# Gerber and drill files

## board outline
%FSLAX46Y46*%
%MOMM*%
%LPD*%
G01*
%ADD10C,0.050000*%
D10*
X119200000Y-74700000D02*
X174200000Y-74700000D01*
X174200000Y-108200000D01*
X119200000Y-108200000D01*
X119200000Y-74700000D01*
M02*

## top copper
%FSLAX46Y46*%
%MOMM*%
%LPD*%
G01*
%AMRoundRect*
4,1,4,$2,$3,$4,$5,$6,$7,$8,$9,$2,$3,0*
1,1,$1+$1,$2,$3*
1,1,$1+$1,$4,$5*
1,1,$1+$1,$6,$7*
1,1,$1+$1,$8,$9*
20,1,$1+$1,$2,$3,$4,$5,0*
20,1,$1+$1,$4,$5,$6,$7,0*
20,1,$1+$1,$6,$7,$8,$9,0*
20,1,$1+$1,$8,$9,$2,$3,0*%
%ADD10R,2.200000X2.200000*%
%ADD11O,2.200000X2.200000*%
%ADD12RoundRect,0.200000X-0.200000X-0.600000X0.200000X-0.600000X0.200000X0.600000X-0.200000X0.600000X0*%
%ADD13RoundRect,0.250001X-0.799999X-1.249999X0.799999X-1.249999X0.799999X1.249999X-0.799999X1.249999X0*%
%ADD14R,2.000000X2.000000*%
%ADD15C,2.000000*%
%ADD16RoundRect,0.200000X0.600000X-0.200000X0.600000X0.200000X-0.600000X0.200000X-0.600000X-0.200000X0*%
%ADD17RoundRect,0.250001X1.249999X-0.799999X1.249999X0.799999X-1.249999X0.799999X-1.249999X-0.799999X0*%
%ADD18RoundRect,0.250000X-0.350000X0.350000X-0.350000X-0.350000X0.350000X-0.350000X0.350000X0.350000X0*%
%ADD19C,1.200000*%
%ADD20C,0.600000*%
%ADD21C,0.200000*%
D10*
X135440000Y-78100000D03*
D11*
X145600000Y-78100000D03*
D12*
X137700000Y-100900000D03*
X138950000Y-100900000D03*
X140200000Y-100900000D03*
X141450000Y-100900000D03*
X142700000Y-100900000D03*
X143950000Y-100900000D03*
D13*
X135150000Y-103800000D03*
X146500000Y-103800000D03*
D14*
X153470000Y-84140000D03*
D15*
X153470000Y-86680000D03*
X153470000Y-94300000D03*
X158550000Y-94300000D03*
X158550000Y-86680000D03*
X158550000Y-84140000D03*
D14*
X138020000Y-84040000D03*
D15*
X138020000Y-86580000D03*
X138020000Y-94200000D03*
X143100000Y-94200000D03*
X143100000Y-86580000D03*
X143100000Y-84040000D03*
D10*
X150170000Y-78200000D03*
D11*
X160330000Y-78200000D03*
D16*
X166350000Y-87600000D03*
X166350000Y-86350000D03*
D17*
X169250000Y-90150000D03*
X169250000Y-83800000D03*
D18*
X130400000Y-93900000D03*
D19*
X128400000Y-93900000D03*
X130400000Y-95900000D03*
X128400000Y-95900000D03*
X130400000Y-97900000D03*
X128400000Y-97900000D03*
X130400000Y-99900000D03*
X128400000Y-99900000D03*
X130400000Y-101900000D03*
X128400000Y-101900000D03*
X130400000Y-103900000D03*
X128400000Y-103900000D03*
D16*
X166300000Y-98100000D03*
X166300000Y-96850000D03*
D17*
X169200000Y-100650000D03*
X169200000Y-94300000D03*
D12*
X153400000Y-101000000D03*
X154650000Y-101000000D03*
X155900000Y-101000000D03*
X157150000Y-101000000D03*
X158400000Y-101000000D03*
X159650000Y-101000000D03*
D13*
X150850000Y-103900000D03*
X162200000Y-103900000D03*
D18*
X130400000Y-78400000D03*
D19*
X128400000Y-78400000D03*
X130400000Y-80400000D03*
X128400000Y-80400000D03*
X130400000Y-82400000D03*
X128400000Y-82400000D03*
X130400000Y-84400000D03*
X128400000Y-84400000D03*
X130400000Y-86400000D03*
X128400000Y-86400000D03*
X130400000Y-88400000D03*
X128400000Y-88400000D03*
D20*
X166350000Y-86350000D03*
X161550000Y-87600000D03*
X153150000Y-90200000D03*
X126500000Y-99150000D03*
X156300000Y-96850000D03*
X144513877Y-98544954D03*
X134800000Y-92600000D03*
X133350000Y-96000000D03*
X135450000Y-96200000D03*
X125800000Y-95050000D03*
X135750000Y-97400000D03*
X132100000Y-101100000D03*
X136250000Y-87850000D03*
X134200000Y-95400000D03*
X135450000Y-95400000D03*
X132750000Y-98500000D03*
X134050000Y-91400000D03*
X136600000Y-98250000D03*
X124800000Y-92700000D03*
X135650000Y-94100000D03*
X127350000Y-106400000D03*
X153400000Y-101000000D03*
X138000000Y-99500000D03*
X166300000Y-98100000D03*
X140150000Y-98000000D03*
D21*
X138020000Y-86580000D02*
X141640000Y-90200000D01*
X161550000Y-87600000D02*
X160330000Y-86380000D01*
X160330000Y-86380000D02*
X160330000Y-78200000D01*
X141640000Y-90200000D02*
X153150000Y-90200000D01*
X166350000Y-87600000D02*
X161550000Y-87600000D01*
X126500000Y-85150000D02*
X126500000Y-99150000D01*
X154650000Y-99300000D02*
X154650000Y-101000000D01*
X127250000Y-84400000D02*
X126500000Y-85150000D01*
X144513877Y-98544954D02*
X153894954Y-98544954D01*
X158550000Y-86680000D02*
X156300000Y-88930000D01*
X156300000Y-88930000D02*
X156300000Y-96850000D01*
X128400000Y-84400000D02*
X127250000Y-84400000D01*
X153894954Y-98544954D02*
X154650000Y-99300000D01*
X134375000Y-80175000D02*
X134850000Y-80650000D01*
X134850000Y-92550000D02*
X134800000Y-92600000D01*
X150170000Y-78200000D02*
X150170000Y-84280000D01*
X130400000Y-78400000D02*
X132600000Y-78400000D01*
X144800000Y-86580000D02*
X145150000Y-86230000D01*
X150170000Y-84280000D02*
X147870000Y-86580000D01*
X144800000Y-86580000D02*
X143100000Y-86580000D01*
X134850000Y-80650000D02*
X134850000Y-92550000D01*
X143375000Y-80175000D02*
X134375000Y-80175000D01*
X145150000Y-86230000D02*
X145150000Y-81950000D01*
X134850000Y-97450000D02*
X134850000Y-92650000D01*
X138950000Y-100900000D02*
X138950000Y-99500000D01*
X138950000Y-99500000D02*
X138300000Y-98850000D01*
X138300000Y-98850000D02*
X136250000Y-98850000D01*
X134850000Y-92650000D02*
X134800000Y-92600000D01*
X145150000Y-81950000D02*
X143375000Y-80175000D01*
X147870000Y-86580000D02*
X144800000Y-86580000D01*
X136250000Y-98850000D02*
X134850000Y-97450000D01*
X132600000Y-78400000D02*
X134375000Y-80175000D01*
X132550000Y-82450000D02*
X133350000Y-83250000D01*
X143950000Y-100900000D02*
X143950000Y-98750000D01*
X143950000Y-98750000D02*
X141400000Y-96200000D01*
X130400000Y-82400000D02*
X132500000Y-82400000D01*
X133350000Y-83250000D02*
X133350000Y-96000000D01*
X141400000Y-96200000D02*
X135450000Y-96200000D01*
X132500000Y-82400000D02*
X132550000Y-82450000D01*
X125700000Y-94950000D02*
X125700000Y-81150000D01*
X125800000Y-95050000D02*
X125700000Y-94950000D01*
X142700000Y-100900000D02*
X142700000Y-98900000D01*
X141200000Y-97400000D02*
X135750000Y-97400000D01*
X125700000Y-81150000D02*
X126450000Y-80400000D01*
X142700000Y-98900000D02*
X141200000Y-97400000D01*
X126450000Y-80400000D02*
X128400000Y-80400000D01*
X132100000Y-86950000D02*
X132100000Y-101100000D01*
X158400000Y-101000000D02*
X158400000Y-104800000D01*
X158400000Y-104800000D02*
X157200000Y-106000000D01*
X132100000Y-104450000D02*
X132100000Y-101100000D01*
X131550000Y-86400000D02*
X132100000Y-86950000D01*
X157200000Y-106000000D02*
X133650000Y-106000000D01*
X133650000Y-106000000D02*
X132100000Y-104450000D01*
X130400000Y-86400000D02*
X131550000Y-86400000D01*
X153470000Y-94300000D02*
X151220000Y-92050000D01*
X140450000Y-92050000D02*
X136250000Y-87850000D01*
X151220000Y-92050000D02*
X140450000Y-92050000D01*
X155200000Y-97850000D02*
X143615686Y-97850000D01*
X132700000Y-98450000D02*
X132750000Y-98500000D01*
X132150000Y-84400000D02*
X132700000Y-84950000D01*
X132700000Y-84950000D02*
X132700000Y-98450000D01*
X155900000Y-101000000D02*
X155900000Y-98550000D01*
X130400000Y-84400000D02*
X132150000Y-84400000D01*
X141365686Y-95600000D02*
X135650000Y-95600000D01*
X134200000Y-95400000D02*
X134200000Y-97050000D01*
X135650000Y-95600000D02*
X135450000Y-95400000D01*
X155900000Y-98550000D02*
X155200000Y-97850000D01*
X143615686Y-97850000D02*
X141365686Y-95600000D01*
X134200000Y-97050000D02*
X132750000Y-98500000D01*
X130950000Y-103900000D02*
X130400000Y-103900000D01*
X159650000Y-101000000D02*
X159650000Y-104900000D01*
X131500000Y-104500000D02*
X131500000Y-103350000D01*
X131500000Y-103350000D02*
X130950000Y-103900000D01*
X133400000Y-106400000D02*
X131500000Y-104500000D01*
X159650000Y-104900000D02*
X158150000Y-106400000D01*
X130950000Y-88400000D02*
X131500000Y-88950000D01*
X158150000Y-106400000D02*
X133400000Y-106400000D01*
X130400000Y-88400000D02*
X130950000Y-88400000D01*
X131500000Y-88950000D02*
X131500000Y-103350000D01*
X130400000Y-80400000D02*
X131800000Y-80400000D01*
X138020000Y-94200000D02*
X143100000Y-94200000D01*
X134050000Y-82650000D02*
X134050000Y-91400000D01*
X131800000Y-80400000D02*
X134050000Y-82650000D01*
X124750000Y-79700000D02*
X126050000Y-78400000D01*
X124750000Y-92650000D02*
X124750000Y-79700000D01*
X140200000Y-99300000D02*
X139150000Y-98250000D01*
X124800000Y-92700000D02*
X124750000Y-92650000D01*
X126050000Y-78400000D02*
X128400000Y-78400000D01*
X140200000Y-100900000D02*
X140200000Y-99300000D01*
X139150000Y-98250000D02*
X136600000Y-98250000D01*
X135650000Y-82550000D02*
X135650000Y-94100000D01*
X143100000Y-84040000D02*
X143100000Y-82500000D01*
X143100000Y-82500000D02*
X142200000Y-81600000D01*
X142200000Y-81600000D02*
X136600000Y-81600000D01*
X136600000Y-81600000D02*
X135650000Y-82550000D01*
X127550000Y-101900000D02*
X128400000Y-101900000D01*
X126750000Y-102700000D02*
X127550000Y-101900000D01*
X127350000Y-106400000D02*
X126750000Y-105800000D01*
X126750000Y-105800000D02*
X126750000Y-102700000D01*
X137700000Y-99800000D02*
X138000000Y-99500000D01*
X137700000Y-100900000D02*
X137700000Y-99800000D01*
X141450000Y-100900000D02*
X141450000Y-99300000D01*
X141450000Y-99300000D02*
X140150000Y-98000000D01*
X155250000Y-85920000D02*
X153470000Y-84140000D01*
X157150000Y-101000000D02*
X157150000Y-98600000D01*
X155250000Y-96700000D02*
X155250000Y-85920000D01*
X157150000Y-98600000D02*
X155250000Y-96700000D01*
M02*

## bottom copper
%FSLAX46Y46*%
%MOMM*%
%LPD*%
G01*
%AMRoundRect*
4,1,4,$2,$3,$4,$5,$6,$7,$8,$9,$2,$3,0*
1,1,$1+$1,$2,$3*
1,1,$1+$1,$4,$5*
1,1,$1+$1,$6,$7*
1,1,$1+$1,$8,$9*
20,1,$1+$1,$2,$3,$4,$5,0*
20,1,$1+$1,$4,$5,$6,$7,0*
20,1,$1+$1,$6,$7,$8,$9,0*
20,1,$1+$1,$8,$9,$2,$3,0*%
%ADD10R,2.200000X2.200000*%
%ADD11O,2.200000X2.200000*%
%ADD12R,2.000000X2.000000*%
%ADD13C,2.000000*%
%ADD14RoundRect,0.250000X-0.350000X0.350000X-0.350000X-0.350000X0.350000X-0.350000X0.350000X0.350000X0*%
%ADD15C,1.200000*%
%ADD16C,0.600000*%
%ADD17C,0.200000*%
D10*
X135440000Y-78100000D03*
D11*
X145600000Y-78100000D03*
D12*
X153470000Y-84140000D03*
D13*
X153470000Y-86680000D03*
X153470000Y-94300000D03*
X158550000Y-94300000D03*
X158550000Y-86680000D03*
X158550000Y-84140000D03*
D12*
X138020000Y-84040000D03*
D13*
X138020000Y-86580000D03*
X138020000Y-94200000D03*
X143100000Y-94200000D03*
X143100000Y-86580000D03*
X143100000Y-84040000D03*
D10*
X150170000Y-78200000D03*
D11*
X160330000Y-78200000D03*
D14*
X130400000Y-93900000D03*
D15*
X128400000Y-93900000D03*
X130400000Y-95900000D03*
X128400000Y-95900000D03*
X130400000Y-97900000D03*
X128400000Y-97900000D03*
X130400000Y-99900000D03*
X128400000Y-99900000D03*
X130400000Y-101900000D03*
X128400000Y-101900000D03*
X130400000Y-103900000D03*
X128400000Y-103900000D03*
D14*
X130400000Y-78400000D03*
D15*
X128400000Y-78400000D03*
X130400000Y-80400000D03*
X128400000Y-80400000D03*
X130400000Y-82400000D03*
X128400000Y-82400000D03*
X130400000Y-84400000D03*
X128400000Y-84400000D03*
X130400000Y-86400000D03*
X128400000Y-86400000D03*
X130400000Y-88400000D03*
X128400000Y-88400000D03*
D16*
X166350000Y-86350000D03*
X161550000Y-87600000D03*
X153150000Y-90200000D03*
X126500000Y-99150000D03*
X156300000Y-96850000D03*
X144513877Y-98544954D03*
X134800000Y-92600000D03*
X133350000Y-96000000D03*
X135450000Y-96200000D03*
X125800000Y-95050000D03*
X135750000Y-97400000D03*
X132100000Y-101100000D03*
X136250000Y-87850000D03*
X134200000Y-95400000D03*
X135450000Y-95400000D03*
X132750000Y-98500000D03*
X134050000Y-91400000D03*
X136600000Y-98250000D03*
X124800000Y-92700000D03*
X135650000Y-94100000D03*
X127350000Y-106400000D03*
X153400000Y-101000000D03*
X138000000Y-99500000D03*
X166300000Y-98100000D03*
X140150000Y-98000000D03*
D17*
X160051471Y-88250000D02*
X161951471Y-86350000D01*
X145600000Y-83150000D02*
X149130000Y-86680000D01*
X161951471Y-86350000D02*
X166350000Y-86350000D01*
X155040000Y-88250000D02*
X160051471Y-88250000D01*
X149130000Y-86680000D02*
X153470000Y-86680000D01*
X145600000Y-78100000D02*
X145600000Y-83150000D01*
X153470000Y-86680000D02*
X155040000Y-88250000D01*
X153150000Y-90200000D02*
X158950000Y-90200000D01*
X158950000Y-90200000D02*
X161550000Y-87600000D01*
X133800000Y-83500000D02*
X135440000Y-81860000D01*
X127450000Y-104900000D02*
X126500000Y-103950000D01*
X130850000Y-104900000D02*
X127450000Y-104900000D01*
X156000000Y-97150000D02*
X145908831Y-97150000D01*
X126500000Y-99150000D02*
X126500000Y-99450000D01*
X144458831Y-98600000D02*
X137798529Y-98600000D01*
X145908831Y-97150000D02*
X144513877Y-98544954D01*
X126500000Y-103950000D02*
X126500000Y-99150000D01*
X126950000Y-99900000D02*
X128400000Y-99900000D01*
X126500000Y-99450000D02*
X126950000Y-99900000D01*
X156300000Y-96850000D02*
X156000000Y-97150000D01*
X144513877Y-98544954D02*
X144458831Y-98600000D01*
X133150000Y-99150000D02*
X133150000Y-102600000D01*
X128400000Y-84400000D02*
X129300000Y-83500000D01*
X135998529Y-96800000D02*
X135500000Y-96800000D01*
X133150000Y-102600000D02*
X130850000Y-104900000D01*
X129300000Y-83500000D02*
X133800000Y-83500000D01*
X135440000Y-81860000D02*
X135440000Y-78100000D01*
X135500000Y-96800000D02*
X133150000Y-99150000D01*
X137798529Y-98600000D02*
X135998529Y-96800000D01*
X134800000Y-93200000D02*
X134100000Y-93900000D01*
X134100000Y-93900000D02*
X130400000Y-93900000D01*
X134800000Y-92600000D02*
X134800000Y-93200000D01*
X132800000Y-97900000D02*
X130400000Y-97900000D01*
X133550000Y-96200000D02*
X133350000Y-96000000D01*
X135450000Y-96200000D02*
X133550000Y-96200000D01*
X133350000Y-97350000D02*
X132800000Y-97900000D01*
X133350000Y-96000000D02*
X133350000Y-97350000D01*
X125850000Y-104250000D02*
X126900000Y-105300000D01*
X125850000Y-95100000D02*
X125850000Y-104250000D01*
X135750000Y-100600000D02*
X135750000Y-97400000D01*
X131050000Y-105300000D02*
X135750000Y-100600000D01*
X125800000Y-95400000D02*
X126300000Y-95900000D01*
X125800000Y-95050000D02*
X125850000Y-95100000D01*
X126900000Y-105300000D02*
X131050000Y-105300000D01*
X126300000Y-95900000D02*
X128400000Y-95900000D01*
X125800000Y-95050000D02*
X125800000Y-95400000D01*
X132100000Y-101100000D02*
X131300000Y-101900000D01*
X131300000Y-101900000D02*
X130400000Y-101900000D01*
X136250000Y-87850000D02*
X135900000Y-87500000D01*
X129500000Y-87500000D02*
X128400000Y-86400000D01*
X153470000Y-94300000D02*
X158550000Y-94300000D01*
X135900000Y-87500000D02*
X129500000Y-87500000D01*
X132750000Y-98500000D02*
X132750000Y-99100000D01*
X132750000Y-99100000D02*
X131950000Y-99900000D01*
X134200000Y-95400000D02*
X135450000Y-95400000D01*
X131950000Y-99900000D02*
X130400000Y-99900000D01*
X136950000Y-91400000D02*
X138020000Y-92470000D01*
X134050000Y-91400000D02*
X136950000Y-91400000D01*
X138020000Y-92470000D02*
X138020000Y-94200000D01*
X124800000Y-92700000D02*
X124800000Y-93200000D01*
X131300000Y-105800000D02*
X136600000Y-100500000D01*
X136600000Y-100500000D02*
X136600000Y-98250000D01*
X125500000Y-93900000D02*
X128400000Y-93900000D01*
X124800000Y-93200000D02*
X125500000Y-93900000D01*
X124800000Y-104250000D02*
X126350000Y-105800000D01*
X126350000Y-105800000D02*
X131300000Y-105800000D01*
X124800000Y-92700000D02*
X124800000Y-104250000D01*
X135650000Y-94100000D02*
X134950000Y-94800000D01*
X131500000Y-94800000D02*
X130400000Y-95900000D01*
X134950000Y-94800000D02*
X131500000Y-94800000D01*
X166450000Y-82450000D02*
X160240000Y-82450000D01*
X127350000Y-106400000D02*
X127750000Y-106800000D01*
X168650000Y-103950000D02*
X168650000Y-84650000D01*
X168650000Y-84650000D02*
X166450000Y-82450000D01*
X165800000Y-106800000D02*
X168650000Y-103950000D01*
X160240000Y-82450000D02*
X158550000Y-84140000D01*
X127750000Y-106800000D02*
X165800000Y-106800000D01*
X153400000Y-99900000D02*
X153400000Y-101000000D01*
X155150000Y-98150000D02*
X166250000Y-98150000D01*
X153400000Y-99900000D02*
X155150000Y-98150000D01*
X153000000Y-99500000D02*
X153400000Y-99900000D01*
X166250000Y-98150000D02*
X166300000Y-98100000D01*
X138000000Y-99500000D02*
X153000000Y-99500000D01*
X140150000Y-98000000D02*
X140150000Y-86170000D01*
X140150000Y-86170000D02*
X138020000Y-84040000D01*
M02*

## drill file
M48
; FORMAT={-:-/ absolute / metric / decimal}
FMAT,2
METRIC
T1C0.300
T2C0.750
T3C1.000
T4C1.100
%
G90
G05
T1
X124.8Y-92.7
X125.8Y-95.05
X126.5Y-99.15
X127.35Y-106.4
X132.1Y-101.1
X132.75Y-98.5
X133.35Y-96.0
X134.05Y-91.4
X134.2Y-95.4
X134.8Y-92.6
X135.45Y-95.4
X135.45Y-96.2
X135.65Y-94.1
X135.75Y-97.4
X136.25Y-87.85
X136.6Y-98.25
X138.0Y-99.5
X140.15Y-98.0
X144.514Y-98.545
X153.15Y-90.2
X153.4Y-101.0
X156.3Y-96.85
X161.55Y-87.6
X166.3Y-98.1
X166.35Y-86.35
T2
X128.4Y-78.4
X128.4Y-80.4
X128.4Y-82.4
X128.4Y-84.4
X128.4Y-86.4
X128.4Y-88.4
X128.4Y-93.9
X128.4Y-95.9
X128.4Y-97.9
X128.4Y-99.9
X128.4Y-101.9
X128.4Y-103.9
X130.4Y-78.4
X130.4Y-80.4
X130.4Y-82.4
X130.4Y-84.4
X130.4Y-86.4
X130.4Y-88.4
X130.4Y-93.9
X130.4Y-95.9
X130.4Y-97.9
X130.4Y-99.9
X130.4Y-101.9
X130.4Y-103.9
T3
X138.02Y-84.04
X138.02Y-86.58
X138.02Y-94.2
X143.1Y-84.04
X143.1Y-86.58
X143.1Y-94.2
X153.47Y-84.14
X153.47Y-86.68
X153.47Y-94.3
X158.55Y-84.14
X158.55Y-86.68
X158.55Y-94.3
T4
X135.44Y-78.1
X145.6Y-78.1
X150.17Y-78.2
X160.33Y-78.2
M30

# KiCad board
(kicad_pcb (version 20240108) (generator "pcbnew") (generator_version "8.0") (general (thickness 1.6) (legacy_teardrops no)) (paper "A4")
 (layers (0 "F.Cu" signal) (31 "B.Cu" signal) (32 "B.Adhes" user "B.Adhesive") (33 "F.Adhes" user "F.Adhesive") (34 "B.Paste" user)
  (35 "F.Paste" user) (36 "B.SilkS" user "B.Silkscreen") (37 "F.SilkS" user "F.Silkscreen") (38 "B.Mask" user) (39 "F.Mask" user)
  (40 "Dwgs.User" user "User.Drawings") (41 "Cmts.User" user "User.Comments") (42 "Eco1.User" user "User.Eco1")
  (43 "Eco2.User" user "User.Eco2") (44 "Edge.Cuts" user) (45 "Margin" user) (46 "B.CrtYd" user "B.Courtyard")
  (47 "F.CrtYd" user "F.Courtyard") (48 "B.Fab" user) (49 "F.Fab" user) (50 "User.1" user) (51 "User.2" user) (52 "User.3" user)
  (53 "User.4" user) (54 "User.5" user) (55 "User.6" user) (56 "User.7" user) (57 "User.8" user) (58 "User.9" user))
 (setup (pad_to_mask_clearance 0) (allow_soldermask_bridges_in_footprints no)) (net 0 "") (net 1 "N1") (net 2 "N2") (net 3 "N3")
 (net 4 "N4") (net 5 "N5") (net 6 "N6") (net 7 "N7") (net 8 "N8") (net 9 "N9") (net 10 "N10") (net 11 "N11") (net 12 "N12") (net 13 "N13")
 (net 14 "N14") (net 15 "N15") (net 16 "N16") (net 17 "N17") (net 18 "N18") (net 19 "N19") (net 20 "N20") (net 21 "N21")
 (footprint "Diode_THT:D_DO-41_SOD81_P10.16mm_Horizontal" (layer "F.Cu") (at 135.44 78.1)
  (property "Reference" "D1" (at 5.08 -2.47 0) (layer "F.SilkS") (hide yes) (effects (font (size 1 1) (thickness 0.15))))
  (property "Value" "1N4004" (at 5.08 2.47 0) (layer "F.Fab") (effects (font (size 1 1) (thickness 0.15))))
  (pad "1" thru_hole rect (at 0 0) (size 2.2 2.2) (drill 1.1) (layers "*.Cu" "*.Mask") (remove_unused_layers no) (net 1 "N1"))
  (pad "2" thru_hole oval (at 10.16 0) (size 2.2 2.2) (drill 1.1) (layers "*.Cu" "*.Mask") (remove_unused_layers no) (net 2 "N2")))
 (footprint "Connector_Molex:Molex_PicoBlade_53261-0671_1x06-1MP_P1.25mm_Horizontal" (layer "F.Cu") (at 140.825 103.3)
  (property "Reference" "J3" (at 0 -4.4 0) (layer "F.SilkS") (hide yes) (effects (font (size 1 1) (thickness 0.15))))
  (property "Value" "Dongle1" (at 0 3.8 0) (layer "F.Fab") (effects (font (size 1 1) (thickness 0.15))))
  (pad "1" smd roundrect (at -3.125 -2.4) (size 0.8 1.6) (layers "F.Cu" "F.Paste" "F.Mask") (roundrect_rratio 0.25) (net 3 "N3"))
  (pad "2" smd roundrect (at -1.875 -2.4) (size 0.8 1.6) (layers "F.Cu" "F.Paste" "F.Mask") (roundrect_rratio 0.25) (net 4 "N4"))
  (pad "3" smd roundrect (at -0.625 -2.4) (size 0.8 1.6) (layers "F.Cu" "F.Paste" "F.Mask") (roundrect_rratio 0.25) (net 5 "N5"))
  (pad "4" smd roundrect (at 0.625 -2.4) (size 0.8 1.6) (layers "F.Cu" "F.Paste" "F.Mask") (roundrect_rratio 0.25) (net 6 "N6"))
  (pad "5" smd roundrect (at 1.875 -2.4) (size 0.8 1.6) (layers "F.Cu" "F.Paste" "F.Mask") (roundrect_rratio 0.25) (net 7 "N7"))
  (pad "6" smd roundrect (at 3.125 -2.4) (size 0.8 1.6) (layers "F.Cu" "F.Paste" "F.Mask") (roundrect_rratio 0.25) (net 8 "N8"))
  (pad "MP" smd roundrect (at -5.675 0.5) (size 2.1 3) (layers "F.Cu" "F.Paste" "F.Mask") (roundrect_rratio 0.119048))
  (pad "MP" smd roundrect (at 5.675 0.5) (size 2.1 3) (layers "F.Cu" "F.Paste" "F.Mask") (roundrect_rratio 0.119048)))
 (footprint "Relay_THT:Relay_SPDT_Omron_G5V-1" (layer "F.Cu") (at 153.47 84.14)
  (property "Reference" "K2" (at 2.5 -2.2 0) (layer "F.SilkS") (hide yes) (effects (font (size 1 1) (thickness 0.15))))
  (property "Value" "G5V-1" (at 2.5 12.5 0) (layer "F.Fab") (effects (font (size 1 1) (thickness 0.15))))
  (pad "1" thru_hole rect (at 0 0) (size 2 2) (drill 1) (layers "*.Cu" "*.Mask") (remove_unused_layers no) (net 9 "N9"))
  (pad "2" thru_hole circle (at 0 2.54) (size 2 2) (drill 1) (layers "*.Cu" "*.Mask") (remove_unused_layers no) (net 2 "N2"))
  (pad "5" thru_hole circle (at 0 10.16) (size 2 2) (drill 1) (layers "*.Cu" "*.Mask") (remove_unused_layers no) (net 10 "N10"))
  (pad "6" thru_hole circle (at 5.08 10.16) (size 2 2) (drill 1) (layers "*.Cu" "*.Mask") (remove_unused_layers no) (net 10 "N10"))
  (pad "9" thru_hole circle (at 5.08 2.54) (size 2 2) (drill 1) (layers "*.Cu" "*.Mask") (remove_unused_layers no) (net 1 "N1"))
  (pad "10" thru_hole circle (at 5.08 0) (size 2 2) (drill 1) (layers "*.Cu" "*.Mask") (remove_unused_layers no) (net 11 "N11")))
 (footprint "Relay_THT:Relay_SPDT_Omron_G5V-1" (layer "F.Cu") (at 138.02 84.04)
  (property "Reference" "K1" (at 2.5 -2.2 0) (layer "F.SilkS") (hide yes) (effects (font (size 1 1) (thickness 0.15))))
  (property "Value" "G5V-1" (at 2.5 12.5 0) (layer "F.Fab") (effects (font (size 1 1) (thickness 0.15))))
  (pad "1" thru_hole rect (at 0 0) (size 2 2) (drill 1) (layers "*.Cu" "*.Mask") (remove_unused_layers no) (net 6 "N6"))
  (pad "2" thru_hole circle (at 0 2.54) (size 2 2) (drill 1) (layers "*.Cu" "*.Mask") (remove_unused_layers no) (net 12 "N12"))
  (pad "5" thru_hole circle (at 0 10.16) (size 2 2) (drill 1) (layers "*.Cu" "*.Mask") (remove_unused_layers no) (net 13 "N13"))
  (pad "6" thru_hole circle (at 5.08 10.16) (size 2 2) (drill 1) (layers "*.Cu" "*.Mask") (remove_unused_layers no) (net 13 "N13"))
  (pad "9" thru_hole circle (at 5.08 2.54) (size 2 2) (drill 1) (layers "*.Cu" "*.Mask") (remove_unused_layers no) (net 4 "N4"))
  (pad "10" thru_hole circle (at 5.08 0) (size 2 2) (drill 1) (layers "*.Cu" "*.Mask") (remove_unused_layers no) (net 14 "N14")))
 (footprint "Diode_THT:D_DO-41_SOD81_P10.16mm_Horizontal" (layer "F.Cu") (at 150.17 78.2)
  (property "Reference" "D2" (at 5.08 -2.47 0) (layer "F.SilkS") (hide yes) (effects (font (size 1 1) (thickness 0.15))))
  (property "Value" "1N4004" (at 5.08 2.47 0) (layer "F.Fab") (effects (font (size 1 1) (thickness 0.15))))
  (pad "1" thru_hole rect (at 0 0) (size 2.2 2.2) (drill 1.1) (layers "*.Cu" "*.Mask") (remove_unused_layers no) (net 4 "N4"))
  (pad "2" thru_hole oval (at 10.16 0) (size 2.2 2.2) (drill 1.1) (layers "*.Cu" "*.Mask") (remove_unused_layers no) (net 12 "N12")))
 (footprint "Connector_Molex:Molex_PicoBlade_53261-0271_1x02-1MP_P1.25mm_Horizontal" (layer "F.Cu") (at 168.75 86.975 90)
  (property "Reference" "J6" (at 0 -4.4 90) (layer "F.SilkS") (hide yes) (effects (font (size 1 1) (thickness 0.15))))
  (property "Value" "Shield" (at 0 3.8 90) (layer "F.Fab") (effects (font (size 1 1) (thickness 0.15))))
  (pad "1" smd roundrect (at -0.625 -2.4 90) (size 0.8 1.6) (layers "F.Cu" "F.Paste" "F.Mask") (roundrect_rratio 0.25) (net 12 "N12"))
  (pad "2" smd roundrect (at 0.625 -2.4 90) (size 0.8 1.6) (layers "F.Cu" "F.Paste" "F.Mask") (roundrect_rratio 0.25) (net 2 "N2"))
  (pad "MP" smd roundrect (at -3.175 0.5 90) (size 2.1 3) (layers "F.Cu" "F.Paste" "F.Mask") (roundrect_rratio 0.119048))
  (pad "MP" smd roundrect (at 3.175 0.5 90) (size 2.1 3) (layers "F.Cu" "F.Paste" "F.Mask") (roundrect_rratio 0.119048)))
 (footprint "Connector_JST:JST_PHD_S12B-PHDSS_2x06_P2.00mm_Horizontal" (layer "F.Cu") (at 130.4 93.9 -90)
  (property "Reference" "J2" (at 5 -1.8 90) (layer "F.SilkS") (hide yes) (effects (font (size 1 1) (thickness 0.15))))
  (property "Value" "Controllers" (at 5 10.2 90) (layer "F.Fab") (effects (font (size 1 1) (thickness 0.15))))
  (pad "1" thru_hole roundrect (at 0 0 270) (size 1.2 1.2) (drill 0.75) (layers "*.Cu" "*.Mask") (remove_unused_layers no)
   (roundrect_rratio 0.208333) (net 4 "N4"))
  (pad "2" thru_hole circle (at 0 2 270) (size 1.2 1.2) (drill 0.75) (layers "*.Cu" "*.Mask") (remove_unused_layers no) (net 5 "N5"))
  (pad "3" thru_hole circle (at 2 0 270) (size 1.2 1.2) (drill 0.75) (layers "*.Cu" "*.Mask") (remove_unused_layers no) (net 14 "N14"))
  (pad "4" thru_hole circle (at 2 2 270) (size 1.2 1.2) (drill 0.75) (layers "*.Cu" "*.Mask") (remove_unused_layers no) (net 7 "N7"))
  (pad "5" thru_hole circle (at 4 0 270) (size 1.2 1.2) (drill 0.75) (layers "*.Cu" "*.Mask") (remove_unused_layers no) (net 8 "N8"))
  (pad "6" thru_hole circle (at 4 2 270) (size 1.2 1.2) (drill 0.75) (layers "*.Cu" "*.Mask") (remove_unused_layers no) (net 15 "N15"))
  (pad "7" thru_hole circle (at 6 0 270) (size 1.2 1.2) (drill 0.75) (layers "*.Cu" "*.Mask") (remove_unused_layers no) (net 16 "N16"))
  (pad "8" thru_hole circle (at 6 2 270) (size 1.2 1.2) (drill 0.75) (layers "*.Cu" "*.Mask") (remove_unused_layers no) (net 1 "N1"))
  (pad "9" thru_hole circle (at 8 0 270) (size 1.2 1.2) (drill 0.75) (layers "*.Cu" "*.Mask") (remove_unused_layers no) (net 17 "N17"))
  (pad "10" thru_hole circle (at 8 2 270) (size 1.2 1.2) (drill 0.75) (layers "*.Cu" "*.Mask") (remove_unused_layers no) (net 11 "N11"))
  (pad "11" thru_hole circle (at 10 0 270) (size 1.2 1.2) (drill 0.75) (layers "*.Cu" "*.Mask") (remove_unused_layers no) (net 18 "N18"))
  (pad "12" thru_hole circle (at 10 2 270) (size 1.2 1.2) (drill 0.75) (layers "*.Cu" "*.Mask") (remove_unused_layers no) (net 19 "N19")))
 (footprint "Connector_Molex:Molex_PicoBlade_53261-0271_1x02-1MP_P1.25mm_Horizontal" (layer "F.Cu") (at 168.7 97.475 90)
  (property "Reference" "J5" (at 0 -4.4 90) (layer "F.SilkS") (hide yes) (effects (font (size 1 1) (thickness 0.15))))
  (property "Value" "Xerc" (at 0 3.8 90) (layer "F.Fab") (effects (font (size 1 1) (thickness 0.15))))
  (pad "1" smd roundrect (at -0.625 -2.4 90) (size 0.8 1.6) (layers "F.Cu" "F.Paste" "F.Mask") (roundrect_rratio 0.25) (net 3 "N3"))
  (pad "2" smd roundrect (at 0.625 -2.4 90) (size 0.8 1.6) (layers "F.Cu" "F.Paste" "F.Mask") (roundrect_rratio 0.25))
  (pad "MP" smd roundrect (at -3.175 0.5 90) (size 2.1 3) (layers "F.Cu" "F.Paste" "F.Mask") (roundrect_rratio 0.119048))
  (pad "MP" smd roundrect (at 3.175 0.5 90) (size 2.1 3) (layers "F.Cu" "F.Paste" "F.Mask") (roundrect_rratio 0.119048)))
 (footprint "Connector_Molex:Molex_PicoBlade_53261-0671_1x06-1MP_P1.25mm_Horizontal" (layer "F.Cu") (at 156.525 103.4)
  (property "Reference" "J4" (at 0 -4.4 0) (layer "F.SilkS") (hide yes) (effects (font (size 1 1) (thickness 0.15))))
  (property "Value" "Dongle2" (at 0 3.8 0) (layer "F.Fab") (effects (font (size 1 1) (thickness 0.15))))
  (pad "1" smd roundrect (at -3.125 -2.4) (size 0.8 1.6) (layers "F.Cu" "F.Paste" "F.Mask") (roundrect_rratio 0.25) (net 3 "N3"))
  (pad "2" smd roundrect (at -1.875 -2.4) (size 0.8 1.6) (layers "F.Cu" "F.Paste" "F.Mask") (roundrect_rratio 0.25) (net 1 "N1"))
  (pad "3" smd roundrect (at -0.625 -2.4) (size 0.8 1.6) (layers "F.Cu" "F.Paste" "F.Mask") (roundrect_rratio 0.25) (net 16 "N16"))
  (pad "4" smd roundrect (at 0.625 -2.4) (size 0.8 1.6) (layers "F.Cu" "F.Paste" "F.Mask") (roundrect_rratio 0.25) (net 9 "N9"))
  (pad "5" smd roundrect (at 1.875 -2.4) (size 0.8 1.6) (layers "F.Cu" "F.Paste" "F.Mask") (roundrect_rratio 0.25) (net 17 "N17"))
  (pad "6" smd roundrect (at 3.125 -2.4) (size 0.8 1.6) (layers "F.Cu" "F.Paste" "F.Mask") (roundrect_rratio 0.25) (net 18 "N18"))
  (pad "MP" smd roundrect (at -5.675 0.5) (size 2.1 3) (layers "F.Cu" "F.Paste" "F.Mask") (roundrect_rratio 0.119048))
  (pad "MP" smd roundrect (at 5.675 0.5) (size 2.1 3) (layers "F.Cu" "F.Paste" "F.Mask") (roundrect_rratio 0.119048)))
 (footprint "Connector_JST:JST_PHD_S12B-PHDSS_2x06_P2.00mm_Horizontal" (layer "F.Cu") (at 130.4 78.4 -90)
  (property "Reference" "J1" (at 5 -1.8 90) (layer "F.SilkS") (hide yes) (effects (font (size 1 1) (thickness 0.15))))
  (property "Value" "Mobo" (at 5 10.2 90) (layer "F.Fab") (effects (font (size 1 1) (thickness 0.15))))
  (pad "1" thru_hole roundrect (at 0 0 270) (size 1.2 1.2) (drill 0.75) (layers "*.Cu" "*.Mask") (remove_unused_layers no)
   (roundrect_rratio 0.208333) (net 4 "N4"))
  (pad "2" thru_hole circle (at 0 2 270) (size 1.2 1.2) (drill 0.75) (layers "*.Cu" "*.Mask") (remove_unused_layers no) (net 5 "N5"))
  (pad "3" thru_hole circle (at 2 0 270) (size 1.2 1.2) (drill 0.75) (layers "*.Cu" "*.Mask") (remove_unused_layers no) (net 13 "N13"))
  (pad "4" thru_hole circle (at 2 2 270) (size 1.2 1.2) (drill 0.75) (layers "*.Cu" "*.Mask") (remove_unused_layers no) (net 7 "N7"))
  (pad "5" thru_hole circle (at 4 0 270) (size 1.2 1.2) (drill 0.75) (layers "*.Cu" "*.Mask") (remove_unused_layers no) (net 8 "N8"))
  (pad "6" thru_hole circle (at 4 2 270) (size 1.2 1.2) (drill 0.75) (layers "*.Cu" "*.Mask") (remove_unused_layers no) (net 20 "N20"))
  (pad "7" thru_hole circle (at 6 0 270) (size 1.2 1.2) (drill 0.75) (layers "*.Cu" "*.Mask") (remove_unused_layers no) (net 16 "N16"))
  (pad "8" thru_hole circle (at 6 2 270) (size 1.2 1.2) (drill 0.75) (layers "*.Cu" "*.Mask") (remove_unused_layers no) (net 1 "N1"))
  (pad "9" thru_hole circle (at 8 0 270) (size 1.2 1.2) (drill 0.75) (layers "*.Cu" "*.Mask") (remove_unused_layers no) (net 17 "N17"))
  (pad "10" thru_hole circle (at 8 2 270) (size 1.2 1.2) (drill 0.75) (layers "*.Cu" "*.Mask") (remove_unused_layers no) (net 10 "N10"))
  (pad "11" thru_hole circle (at 10 0 270) (size 1.2 1.2) (drill 0.75) (layers "*.Cu" "*.Mask") (remove_unused_layers no) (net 18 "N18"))
  (pad "12" thru_hole circle (at 10 2 270) (size 1.2 1.2) (drill 0.75) (layers "*.Cu" "*.Mask") (remove_unused_layers no) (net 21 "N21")))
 (gr_rect (start 119.2 74.7) (end 174.2 108.2) (stroke (width 0.05) (type default)) (fill none) (layer "Edge.Cuts"))
 (via (at 166.35 86.35) (size 0.6) (drill 0.3) (layers "F.Cu" "B.Cu") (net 2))
 (segment (start 160.051471 88.25) (end 161.951471 86.35) (width 0.2) (layer "B.Cu") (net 2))
 (segment (start 145.6 83.15) (end 149.13 86.68) (width 0.2) (layer "B.Cu") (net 2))
 (segment (start 161.951471 86.35) (end 166.35 86.35) (width 0.2) (layer "B.Cu") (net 2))
 (segment (start 155.04 88.25) (end 160.051471 88.25) (width 0.2) (layer "B.Cu") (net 2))
 (segment (start 149.13 86.68) (end 153.47 86.68) (width 0.2) (layer "B.Cu") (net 2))
 (segment (start 145.6 78.1) (end 145.6 83.15) (width 0.2) (layer "B.Cu") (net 2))
 (segment (start 153.47 86.68) (end 155.04 88.25) (width 0.2) (layer "B.Cu") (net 2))
 (segment (start 138.02 86.58) (end 141.64 90.2) (width 0.2) (layer "F.Cu") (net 12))
 (segment (start 161.55 87.6) (end 160.33 86.38) (width 0.2) (layer "F.Cu") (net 12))
 (segment (start 160.33 86.38) (end 160.33 78.2) (width 0.2) (layer "F.Cu") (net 12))
 (segment (start 141.64 90.2) (end 153.15 90.2) (width 0.2) (layer "F.Cu") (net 12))
 (segment (start 166.35 87.6) (end 161.55 87.6) (width 0.2) (layer "F.Cu") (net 12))
 (via (at 161.55 87.6) (size 0.6) (drill 0.3) (layers "F.Cu" "B.Cu") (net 12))
 (via (at 153.15 90.2) (size 0.6) (drill 0.3) (layers "F.Cu" "B.Cu") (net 12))
 (segment (start 153.15 90.2) (end 158.95 90.2) (width 0.2) (layer "B.Cu") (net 12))
 (segment (start 158.95 90.2) (end 161.55 87.6) (width 0.2) (layer "B.Cu") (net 12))
 (segment (start 126.5 85.15) (end 126.5 99.15) (width 0.2) (layer "F.Cu") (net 1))
 (segment (start 154.65 99.3) (end 154.65 101) (width 0.2) (layer "F.Cu") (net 1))
 (segment (start 127.25 84.4) (end 126.5 85.15) (width 0.2) (layer "F.Cu") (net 1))
 (segment (start 144.513877 98.544954) (end 153.894954 98.544954) (width 0.2) (layer "F.Cu") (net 1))
 (segment (start 158.55 86.68) (end 156.3 88.93) (width 0.2) (layer "F.Cu") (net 1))
 (segment (start 156.3 88.93) (end 156.3 96.85) (width 0.2) (layer "F.Cu") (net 1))
 (segment (start 128.4 84.4) (end 127.25 84.4) (width 0.2) (layer "F.Cu") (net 1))
 (segment (start 153.894954 98.544954) (end 154.65 99.3) (width 0.2) (layer "F.Cu") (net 1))
 (via (at 126.5 99.15) (size 0.6) (drill 0.3) (layers "F.Cu" "B.Cu") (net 1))
 (via (at 156.3 96.85) (size 0.6) (drill 0.3) (layers "F.Cu" "B.Cu") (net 1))
 (via (at 144.513877 98.544954) (size 0.6) (drill 0.3) (layers "F.Cu" "B.Cu") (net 1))
 (segment (start 133.8 83.5) (end 135.44 81.86) (width 0.2) (layer "B.Cu") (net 1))
 (segment (start 127.45 104.9) (end 126.5 103.95) (width 0.2) (layer "B.Cu") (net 1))
 (segment (start 130.85 104.9) (end 127.45 104.9) (width 0.2) (layer "B.Cu") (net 1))
 (segment (start 156 97.15) (end 145.908831 97.15) (width 0.2) (layer "B.Cu") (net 1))
 (segment (start 126.5 99.15) (end 126.5 99.45) (width 0.2) (layer "B.Cu") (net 1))
 (segment (start 144.458831 98.6) (end 137.798529 98.6) (width 0.2) (layer "B.Cu") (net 1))
 (segment (start 145.908831 97.15) (end 144.513877 98.544954) (width 0.2) (layer "B.Cu") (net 1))
 (segment (start 126.5 103.95) (end 126.5 99.15) (width 0.2) (layer "B.Cu") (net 1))
 (segment (start 126.95 99.9) (end 128.4 99.9) (width 0.2) (layer "B.Cu") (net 1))
 (segment (start 126.5 99.45) (end 126.95 99.9) (width 0.2) (layer "B.Cu") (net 1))
 (segment (start 156.3 96.85) (end 156 97.15) (width 0.2) (layer "B.Cu") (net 1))
 (segment (start 144.513877 98.544954) (end 144.458831 98.6) (width 0.2) (layer "B.Cu") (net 1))
 (segment (start 133.15 99.15) (end 133.15 102.6) (width 0.2) (layer "B.Cu") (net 1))
 (segment (start 128.4 84.4) (end 129.3 83.5) (width 0.2) (layer "B.Cu") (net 1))
 (segment (start 135.998529 96.8) (end 135.5 96.8) (width 0.2) (layer "B.Cu") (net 1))
 (segment (start 133.15 102.6) (end 130.85 104.9) (width 0.2) (layer "B.Cu") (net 1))
 (segment (start 129.3 83.5) (end 133.8 83.5) (width 0.2) (layer "B.Cu") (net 1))
 (segment (start 135.44 81.86) (end 135.44 78.1) (width 0.2) (layer "B.Cu") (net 1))
 (segment (start 135.5 96.8) (end 133.15 99.15) (width 0.2) (layer "B.Cu") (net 1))
 (segment (start 137.798529 98.6) (end 135.998529 96.8) (width 0.2) (layer "B.Cu") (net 1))
 (segment (start 134.375 80.175) (end 134.85 80.65) (width 0.2) (layer "F.Cu") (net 4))
 (segment (start 134.85 92.55) (end 134.8 92.6) (width 0.2) (layer "F.Cu") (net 4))
 (segment (start 150.17 78.2) (end 150.17 84.28) (width 0.2) (layer "F.Cu") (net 4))
 (segment (start 130.4 78.4) (end 132.6 78.4) (width 0.2) (layer "F.Cu") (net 4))
 (segment (start 144.8 86.58) (end 145.15 86.23) (width 0.2) (layer "F.Cu") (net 4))
 (segment (start 150.17 84.28) (end 147.87 86.58) (width 0.2) (layer "F.Cu") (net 4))
 (segment (start 144.8 86.58) (end 143.1 86.58) (width 0.2) (layer "F.Cu") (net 4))
 (segment (start 134.85 80.65) (end 134.85 92.55) (width 0.2) (layer "F.Cu") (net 4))
 (segment (start 143.375 80.175) (end 134.375 80.175) (width 0.2) (layer "F.Cu") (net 4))
 (segment (start 145.15 86.23) (end 145.15 81.95) (width 0.2) (layer "F.Cu") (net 4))
 (segment (start 134.85 97.45) (end 134.85 92.65) (width 0.2) (layer "F.Cu") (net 4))
 (segment (start 138.95 100.9) (end 138.95 99.5) (width 0.2) (layer "F.Cu") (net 4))
 (segment (start 138.95 99.5) (end 138.3 98.85) (width 0.2) (layer "F.Cu") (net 4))
 (segment (start 138.3 98.85) (end 136.25 98.85) (width 0.2) (layer "F.Cu") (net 4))
 (segment (start 134.85 92.65) (end 134.8 92.6) (width 0.2) (layer "F.Cu") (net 4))
 (segment (start 145.15 81.95) (end 143.375 80.175) (width 0.2) (layer "F.Cu") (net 4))
 (segment (start 147.87 86.58) (end 144.8 86.58) (width 0.2) (layer "F.Cu") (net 4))
 (segment (start 136.25 98.85) (end 134.85 97.45) (width 0.2) (layer "F.Cu") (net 4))
 (segment (start 132.6 78.4) (end 134.375 80.175) (width 0.2) (layer "F.Cu") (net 4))
 (via (at 134.8 92.6) (size 0.6) (drill 0.3) (layers "F.Cu" "B.Cu") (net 4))
 (segment (start 134.8 93.2) (end 134.1 93.9) (width 0.2) (layer "B.Cu") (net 4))
 (segment (start 134.1 93.9) (end 130.4 93.9) (width 0.2) (layer "B.Cu") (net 4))
 (segment (start 134.8 92.6) (end 134.8 93.2) (width 0.2) (layer "B.Cu") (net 4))
 (segment (start 132.55 82.45) (end 133.35 83.25) (width 0.2) (layer "F.Cu") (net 8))
 (segment (start 143.95 100.9) (end 143.95 98.75) (width 0.2) (layer "F.Cu") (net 8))
 (segment (start 143.95 98.75) (end 141.4 96.2) (width 0.2) (layer "F.Cu") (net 8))
 (segment (start 130.4 82.4) (end 132.5 82.4) (width 0.2) (layer "F.Cu") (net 8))
 (segment (start 133.35 83.25) (end 133.35 96) (width 0.2) (layer "F.Cu") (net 8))
 (segment (start 141.4 96.2) (end 135.45 96.2) (width 0.2) (layer "F.Cu") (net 8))
 (segment (start 132.5 82.4) (end 132.55 82.45) (width 0.2) (layer "F.Cu") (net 8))
 (via (at 133.35 96) (size 0.6) (drill 0.3) (layers "F.Cu" "B.Cu") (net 8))
 (via (at 135.45 96.2) (size 0.6) (drill 0.3) (layers "F.Cu" "B.Cu") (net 8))
 (segment (start 132.8 97.9) (end 130.4 97.9) (width 0.2) (layer "B.Cu") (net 8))
 (segment (start 133.55 96.2) (end 133.35 96) (width 0.2) (layer "B.Cu") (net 8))
 (segment (start 135.45 96.2) (end 133.55 96.2) (width 0.2) (layer "B.Cu") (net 8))
 (segment (start 133.35 97.35) (end 132.8 97.9) (width 0.2) (layer "B.Cu") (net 8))
 (segment (start 133.35 96) (end 133.35 97.35) (width 0.2) (layer "B.Cu") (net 8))
 (segment (start 125.7 94.95) (end 125.7 81.15) (width 0.2) (layer "F.Cu") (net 7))
 (segment (start 125.8 95.05) (end 125.7 94.95) (width 0.2) (layer "F.Cu") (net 7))
 (segment (start 142.7 100.9) (end 142.7 98.9) (width 0.2) (layer "F.Cu") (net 7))
 (segment (start 141.2 97.4) (end 135.75 97.4) (width 0.2) (layer "F.Cu") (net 7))
 (segment (start 125.7 81.15) (end 126.45 80.4) (width 0.2) (layer "F.Cu") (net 7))
 (segment (start 142.7 98.9) (end 141.2 97.4) (width 0.2) (layer "F.Cu") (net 7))
 (segment (start 126.45 80.4) (end 128.4 80.4) (width 0.2) (layer "F.Cu") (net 7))
 (via (at 125.8 95.05) (size 0.6) (drill 0.3) (layers "F.Cu" "B.Cu") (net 7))
 (via (at 135.75 97.4) (size 0.6) (drill 0.3) (layers "F.Cu" "B.Cu") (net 7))
 (segment (start 125.85 104.25) (end 126.9 105.3) (width 0.2) (layer "B.Cu") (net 7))
 (segment (start 125.85 95.1) (end 125.85 104.25) (width 0.2) (layer "B.Cu") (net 7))
 (segment (start 135.75 100.6) (end 135.75 97.4) (width 0.2) (layer "B.Cu") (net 7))
 (segment (start 131.05 105.3) (end 135.75 100.6) (width 0.2) (layer "B.Cu") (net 7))
 (segment (start 125.8 95.4) (end 126.3 95.9) (width 0.2) (layer "B.Cu") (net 7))
 (segment (start 125.8 95.05) (end 125.85 95.1) (width 0.2) (layer "B.Cu") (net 7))
 (segment (start 126.9 105.3) (end 131.05 105.3) (width 0.2) (layer "B.Cu") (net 7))
 (segment (start 126.3 95.9) (end 128.4 95.9) (width 0.2) (layer "B.Cu") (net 7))
 (segment (start 125.8 95.05) (end 125.8 95.4) (width 0.2) (layer "B.Cu") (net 7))
 (segment (start 132.1 86.95) (end 132.1 101.1) (width 0.2) (layer "F.Cu") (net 17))
 (segment (start 158.4 101) (end 158.4 104.8) (width 0.2) (layer "F.Cu") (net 17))
 (segment (start 158.4 104.8) (end 157.2 106) (width 0.2) (layer "F.Cu") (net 17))
 (segment (start 132.1 104.45) (end 132.1 101.1) (width 0.2) (layer "F.Cu") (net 17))
 (segment (start 131.55 86.4) (end 132.1 86.95) (width 0.2) (layer "F.Cu") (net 17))
 (segment (start 157.2 106) (end 133.65 106) (width 0.2) (layer "F.Cu") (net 17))
 (segment (start 133.65 106) (end 132.1 104.45) (width 0.2) (layer "F.Cu") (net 17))
 (segment (start 130.4 86.4) (end 131.55 86.4) (width 0.2) (layer "F.Cu") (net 17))
 (via (at 132.1 101.1) (size 0.6) (drill 0.3) (layers "F.Cu" "B.Cu") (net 17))
 (segment (start 132.1 101.1) (end 131.3 101.9) (width 0.2) (layer "B.Cu") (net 17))
 (segment (start 131.3 101.9) (end 130.4 101.9) (width 0.2) (layer "B.Cu") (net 17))
 (segment (start 153.47 94.3) (end 151.22 92.05) (width 0.2) (layer "F.Cu") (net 10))
 (segment (start 140.45 92.05) (end 136.25 87.85) (width 0.2) (layer "F.Cu") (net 10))
 (segment (start 151.22 92.05) (end 140.45 92.05) (width 0.2) (layer "F.Cu") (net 10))
 (via (at 136.25 87.85) (size 0.6) (drill 0.3) (layers "F.Cu" "B.Cu") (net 10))
 (segment (start 136.25 87.85) (end 135.9 87.5) (width 0.2) (layer "B.Cu") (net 10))
 (segment (start 129.5 87.5) (end 128.4 86.4) (width 0.2) (layer "B.Cu") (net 10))
 (segment (start 153.47 94.3) (end 158.55 94.3) (width 0.2) (layer "B.Cu") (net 10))
 (segment (start 135.9 87.5) (end 129.5 87.5) (width 0.2) (layer "B.Cu") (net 10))
 (segment (start 155.2 97.85) (end 143.615686 97.85) (width 0.2) (layer "F.Cu") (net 16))
 (segment (start 132.7 98.45) (end 132.75 98.5) (width 0.2) (layer "F.Cu") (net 16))
 (segment (start 132.15 84.4) (end 132.7 84.95) (width 0.2) (layer "F.Cu") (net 16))
 (segment (start 132.7 84.95) (end 132.7 98.45) (width 0.2) (layer "F.Cu") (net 16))
 (segment (start 155.9 101) (end 155.9 98.55) (width 0.2) (layer "F.Cu") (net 16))
 (segment (start 130.4 84.4) (end 132.15 84.4) (width 0.2) (layer "F.Cu") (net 16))
 (segment (start 141.365686 95.6) (end 135.65 95.6) (width 0.2) (layer "F.Cu") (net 16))
 (segment (start 134.2 95.4) (end 134.2 97.05) (width 0.2) (layer "F.Cu") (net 16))
 (segment (start 135.65 95.6) (end 135.45 95.4) (width 0.2) (layer "F.Cu") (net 16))
 (segment (start 155.9 98.55) (end 155.2 97.85) (width 0.2) (layer "F.Cu") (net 16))
 (segment (start 143.615686 97.85) (end 141.365686 95.6) (width 0.2) (layer "F.Cu") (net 16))
 (segment (start 134.2 97.05) (end 132.75 98.5) (width 0.2) (layer "F.Cu") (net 16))
 (via (at 134.2 95.4) (size 0.6) (drill 0.3) (layers "F.Cu" "B.Cu") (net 16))
 (via (at 135.45 95.4) (size 0.6) (drill 0.3) (layers "F.Cu" "B.Cu") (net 16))
 (via (at 132.75 98.5) (size 0.6) (drill 0.3) (layers "F.Cu" "B.Cu") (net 16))
 (segment (start 132.75 98.5) (end 132.75 99.1) (width 0.2) (layer "B.Cu") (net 16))
 (segment (start 132.75 99.1) (end 131.95 99.9) (width 0.2) (layer "B.Cu") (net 16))
 (segment (start 134.2 95.4) (end 135.45 95.4) (width 0.2) (layer "B.Cu") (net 16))
 (segment (start 131.95 99.9) (end 130.4 99.9) (width 0.2) (layer "B.Cu") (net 16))
 (segment (start 130.95 103.9) (end 130.4 103.9) (width 0.2) (layer "F.Cu") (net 18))
 (segment (start 159.65 101) (end 159.65 104.9) (width 0.2) (layer "F.Cu") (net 18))
 (segment (start 131.5 104.5) (end 131.5 103.35) (width 0.2) (layer "F.Cu") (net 18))
 (segment (start 131.5 103.35) (end 130.95 103.9) (width 0.2) (layer "F.Cu") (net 18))
 (segment (start 133.4 106.4) (end 131.5 104.5) (width 0.2) (layer "F.Cu") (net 18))
 (segment (start 159.65 104.9) (end 158.15 106.4) (width 0.2) (layer "F.Cu") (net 18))
 (segment (start 130.95 88.4) (end 131.5 88.95) (width 0.2) (layer "F.Cu") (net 18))
 (segment (start 158.15 106.4) (end 133.4 106.4) (width 0.2) (layer "F.Cu") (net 18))
 (segment (start 130.4 88.4) (end 130.95 88.4) (width 0.2) (layer "F.Cu") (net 18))
 (segment (start 131.5 88.95) (end 131.5 103.35) (width 0.2) (layer "F.Cu") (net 18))
 (segment (start 130.4 80.4) (end 131.8 80.4) (width 0.2) (layer "F.Cu") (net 13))
 (segment (start 138.02 94.2) (end 143.1 94.2) (width 0.2) (layer "F.Cu") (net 13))
 (segment (start 134.05 82.65) (end 134.05 91.4) (width 0.2) (layer "F.Cu") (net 13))
 (segment (start 131.8 80.4) (end 134.05 82.65) (width 0.2) (layer "F.Cu") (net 13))
 (via (at 134.05 91.4) (size 0.6) (drill 0.3) (layers "F.Cu" "B.Cu") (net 13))
 (segment (start 136.95 91.4) (end 138.02 92.47) (width 0.2) (layer "B.Cu") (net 13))
 (segment (start 134.05 91.4) (end 136.95 91.4) (width 0.2) (layer "B.Cu") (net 13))
 (segment (start 138.02 92.47) (end 138.02 94.2) (width 0.2) (layer "B.Cu") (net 13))
 (segment (start 124.75 79.7) (end 126.05 78.4) (width 0.2) (layer "F.Cu") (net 5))
 (segment (start 124.75 92.65) (end 124.75 79.7) (width 0.2) (layer "F.Cu") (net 5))
 (segment (start 140.2 99.3) (end 139.15 98.25) (width 0.2) (layer "F.Cu") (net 5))
 (segment (start 124.8 92.7) (end 124.75 92.65) (width 0.2) (layer "F.Cu") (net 5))
 (segment (start 126.05 78.4) (end 128.4 78.4) (width 0.2) (layer "F.Cu") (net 5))
 (segment (start 140.2 100.9) (end 140.2 99.3) (width 0.2) (layer "F.Cu") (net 5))
 (segment (start 139.15 98.25) (end 136.6 98.25) (width 0.2) (layer "F.Cu") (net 5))
 (via (at 136.6 98.25) (size 0.6) (drill 0.3) (layers "F.Cu" "B.Cu") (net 5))
 (via (at 124.8 92.7) (size 0.6) (drill 0.3) (layers "F.Cu" "B.Cu") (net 5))
 (segment (start 124.8 92.7) (end 124.8 93.2) (width 0.2) (layer "B.Cu") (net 5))
 (segment (start 131.3 105.8) (end 136.6 100.5) (width 0.2) (layer "B.Cu") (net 5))
 (segment (start 136.6 100.5) (end 136.6 98.25) (width 0.2) (layer "B.Cu") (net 5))
 (segment (start 125.5 93.9) (end 128.4 93.9) (width 0.2) (layer "B.Cu") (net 5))
 (segment (start 124.8 93.2) (end 125.5 93.9) (width 0.2) (layer "B.Cu") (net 5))
 (segment (start 124.8 104.25) (end 126.35 105.8) (width 0.2) (layer "B.Cu") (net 5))
 (segment (start 126.35 105.8) (end 131.3 105.8) (width 0.2) (layer "B.Cu") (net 5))
 (segment (start 124.8 92.7) (end 124.8 104.25) (width 0.2) (layer "B.Cu") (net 5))
 (segment (start 135.65 82.55) (end 135.65 94.1) (width 0.2) (layer "F.Cu") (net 14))
 (segment (start 143.1 84.04) (end 143.1 82.5) (width 0.2) (layer "F.Cu") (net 14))
 (segment (start 143.1 82.5) (end 142.2 81.6) (width 0.2) (layer "F.Cu") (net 14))
 (segment (start 142.2 81.6) (end 136.6 81.6) (width 0.2) (layer "F.Cu") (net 14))
 (segment (start 136.6 81.6) (end 135.65 82.55) (width 0.2) (layer "F.Cu") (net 14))
 (via (at 135.65 94.1) (size 0.6) (drill 0.3) (layers "F.Cu" "B.Cu") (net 14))
 (segment (start 135.65 94.1) (end 134.95 94.8) (width 0.2) (layer "B.Cu") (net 14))
 (segment (start 131.5 94.8) (end 130.4 95.9) (width 0.2) (layer "B.Cu") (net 14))
 (segment (start 134.95 94.8) (end 131.5 94.8) (width 0.2) (layer "B.Cu") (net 14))
 (segment (start 127.55 101.9) (end 128.4 101.9) (width 0.2) (layer "F.Cu") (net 11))
 (segment (start 126.75 102.7) (end 127.55 101.9) (width 0.2) (layer "F.Cu") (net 11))
 (segment (start 127.35 106.4) (end 126.75 105.8) (width 0.2) (layer "F.Cu") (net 11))
 (segment (start 126.75 105.8) (end 126.75 102.7) (width 0.2) (layer "F.Cu") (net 11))
 (via (at 127.35 106.4) (size 0.6) (drill 0.3) (layers "F.Cu" "B.Cu") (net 11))
 (segment (start 166.45 82.45) (end 160.24 82.45) (width 0.2) (layer "B.Cu") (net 11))
 (segment (start 127.35 106.4) (end 127.75 106.8) (width 0.2) (layer "B.Cu") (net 11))
 (segment (start 168.65 103.95) (end 168.65 84.65) (width 0.2) (layer "B.Cu") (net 11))
 (segment (start 168.65 84.65) (end 166.45 82.45) (width 0.2) (layer "B.Cu") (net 11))
 (segment (start 165.8 106.8) (end 168.65 103.95) (width 0.2) (layer "B.Cu") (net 11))
 (segment (start 160.24 82.45) (end 158.55 84.14) (width 0.2) (layer "B.Cu") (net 11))
 (segment (start 127.75 106.8) (end 165.8 106.8) (width 0.2) (layer "B.Cu") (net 11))
 (segment (start 137.7 99.8) (end 138 99.5) (width 0.2) (layer "F.Cu") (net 3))
 (segment (start 137.7 100.9) (end 137.7 99.8) (width 0.2) (layer "F.Cu") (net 3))
 (via (at 153.4 101) (size 0.6) (drill 0.3) (layers "F.Cu" "B.Cu") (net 3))
 (via (at 138 99.5) (size 0.6) (drill 0.3) (layers "F.Cu" "B.Cu") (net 3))
 (via (at 166.3 98.1) (size 0.6) (drill 0.3) (layers "F.Cu" "B.Cu") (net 3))
 (segment (start 153.4 99.9) (end 153.4 101) (width 0.2) (layer "B.Cu") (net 3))
 (segment (start 155.15 98.15) (end 166.25 98.15) (width 0.2) (layer "B.Cu") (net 3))
 (segment (start 153.4 99.9) (end 155.15 98.15) (width 0.2) (layer "B.Cu") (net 3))
 (segment (start 153 99.5) (end 153.4 99.9) (width 0.2) (layer "B.Cu") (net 3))
 (segment (start 166.25 98.15) (end 166.3 98.1) (width 0.2) (layer "B.Cu") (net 3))
 (segment (start 138 99.5) (end 153 99.5) (width 0.2) (layer "B.Cu") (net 3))
 (segment (start 141.45 100.9) (end 141.45 99.3) (width 0.2) (layer "F.Cu") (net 6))
 (segment (start 141.45 99.3) (end 140.15 98) (width 0.2) (layer "F.Cu") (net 6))
 (via (at 140.15 98) (size 0.6) (drill 0.3) (layers "F.Cu" "B.Cu") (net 6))
 (segment (start 140.15 98) (end 140.15 86.17) (width 0.2) (layer "B.Cu") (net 6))
 (segment (start 140.15 86.17) (end 138.02 84.04) (width 0.2) (layer "B.Cu") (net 6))
 (segment (start 155.25 85.92) (end 153.47 84.14) (width 0.2) (layer "F.Cu") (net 9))
 (segment (start 157.15 101) (end 157.15 98.6) (width 0.2) (layer "F.Cu") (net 9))
 (segment (start 155.25 96.7) (end 155.25 85.92) (width 0.2) (layer "F.Cu") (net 9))
 (segment (start 157.15 98.6) (end 155.25 96.7) (width 0.2) (layer "F.Cu") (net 9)))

